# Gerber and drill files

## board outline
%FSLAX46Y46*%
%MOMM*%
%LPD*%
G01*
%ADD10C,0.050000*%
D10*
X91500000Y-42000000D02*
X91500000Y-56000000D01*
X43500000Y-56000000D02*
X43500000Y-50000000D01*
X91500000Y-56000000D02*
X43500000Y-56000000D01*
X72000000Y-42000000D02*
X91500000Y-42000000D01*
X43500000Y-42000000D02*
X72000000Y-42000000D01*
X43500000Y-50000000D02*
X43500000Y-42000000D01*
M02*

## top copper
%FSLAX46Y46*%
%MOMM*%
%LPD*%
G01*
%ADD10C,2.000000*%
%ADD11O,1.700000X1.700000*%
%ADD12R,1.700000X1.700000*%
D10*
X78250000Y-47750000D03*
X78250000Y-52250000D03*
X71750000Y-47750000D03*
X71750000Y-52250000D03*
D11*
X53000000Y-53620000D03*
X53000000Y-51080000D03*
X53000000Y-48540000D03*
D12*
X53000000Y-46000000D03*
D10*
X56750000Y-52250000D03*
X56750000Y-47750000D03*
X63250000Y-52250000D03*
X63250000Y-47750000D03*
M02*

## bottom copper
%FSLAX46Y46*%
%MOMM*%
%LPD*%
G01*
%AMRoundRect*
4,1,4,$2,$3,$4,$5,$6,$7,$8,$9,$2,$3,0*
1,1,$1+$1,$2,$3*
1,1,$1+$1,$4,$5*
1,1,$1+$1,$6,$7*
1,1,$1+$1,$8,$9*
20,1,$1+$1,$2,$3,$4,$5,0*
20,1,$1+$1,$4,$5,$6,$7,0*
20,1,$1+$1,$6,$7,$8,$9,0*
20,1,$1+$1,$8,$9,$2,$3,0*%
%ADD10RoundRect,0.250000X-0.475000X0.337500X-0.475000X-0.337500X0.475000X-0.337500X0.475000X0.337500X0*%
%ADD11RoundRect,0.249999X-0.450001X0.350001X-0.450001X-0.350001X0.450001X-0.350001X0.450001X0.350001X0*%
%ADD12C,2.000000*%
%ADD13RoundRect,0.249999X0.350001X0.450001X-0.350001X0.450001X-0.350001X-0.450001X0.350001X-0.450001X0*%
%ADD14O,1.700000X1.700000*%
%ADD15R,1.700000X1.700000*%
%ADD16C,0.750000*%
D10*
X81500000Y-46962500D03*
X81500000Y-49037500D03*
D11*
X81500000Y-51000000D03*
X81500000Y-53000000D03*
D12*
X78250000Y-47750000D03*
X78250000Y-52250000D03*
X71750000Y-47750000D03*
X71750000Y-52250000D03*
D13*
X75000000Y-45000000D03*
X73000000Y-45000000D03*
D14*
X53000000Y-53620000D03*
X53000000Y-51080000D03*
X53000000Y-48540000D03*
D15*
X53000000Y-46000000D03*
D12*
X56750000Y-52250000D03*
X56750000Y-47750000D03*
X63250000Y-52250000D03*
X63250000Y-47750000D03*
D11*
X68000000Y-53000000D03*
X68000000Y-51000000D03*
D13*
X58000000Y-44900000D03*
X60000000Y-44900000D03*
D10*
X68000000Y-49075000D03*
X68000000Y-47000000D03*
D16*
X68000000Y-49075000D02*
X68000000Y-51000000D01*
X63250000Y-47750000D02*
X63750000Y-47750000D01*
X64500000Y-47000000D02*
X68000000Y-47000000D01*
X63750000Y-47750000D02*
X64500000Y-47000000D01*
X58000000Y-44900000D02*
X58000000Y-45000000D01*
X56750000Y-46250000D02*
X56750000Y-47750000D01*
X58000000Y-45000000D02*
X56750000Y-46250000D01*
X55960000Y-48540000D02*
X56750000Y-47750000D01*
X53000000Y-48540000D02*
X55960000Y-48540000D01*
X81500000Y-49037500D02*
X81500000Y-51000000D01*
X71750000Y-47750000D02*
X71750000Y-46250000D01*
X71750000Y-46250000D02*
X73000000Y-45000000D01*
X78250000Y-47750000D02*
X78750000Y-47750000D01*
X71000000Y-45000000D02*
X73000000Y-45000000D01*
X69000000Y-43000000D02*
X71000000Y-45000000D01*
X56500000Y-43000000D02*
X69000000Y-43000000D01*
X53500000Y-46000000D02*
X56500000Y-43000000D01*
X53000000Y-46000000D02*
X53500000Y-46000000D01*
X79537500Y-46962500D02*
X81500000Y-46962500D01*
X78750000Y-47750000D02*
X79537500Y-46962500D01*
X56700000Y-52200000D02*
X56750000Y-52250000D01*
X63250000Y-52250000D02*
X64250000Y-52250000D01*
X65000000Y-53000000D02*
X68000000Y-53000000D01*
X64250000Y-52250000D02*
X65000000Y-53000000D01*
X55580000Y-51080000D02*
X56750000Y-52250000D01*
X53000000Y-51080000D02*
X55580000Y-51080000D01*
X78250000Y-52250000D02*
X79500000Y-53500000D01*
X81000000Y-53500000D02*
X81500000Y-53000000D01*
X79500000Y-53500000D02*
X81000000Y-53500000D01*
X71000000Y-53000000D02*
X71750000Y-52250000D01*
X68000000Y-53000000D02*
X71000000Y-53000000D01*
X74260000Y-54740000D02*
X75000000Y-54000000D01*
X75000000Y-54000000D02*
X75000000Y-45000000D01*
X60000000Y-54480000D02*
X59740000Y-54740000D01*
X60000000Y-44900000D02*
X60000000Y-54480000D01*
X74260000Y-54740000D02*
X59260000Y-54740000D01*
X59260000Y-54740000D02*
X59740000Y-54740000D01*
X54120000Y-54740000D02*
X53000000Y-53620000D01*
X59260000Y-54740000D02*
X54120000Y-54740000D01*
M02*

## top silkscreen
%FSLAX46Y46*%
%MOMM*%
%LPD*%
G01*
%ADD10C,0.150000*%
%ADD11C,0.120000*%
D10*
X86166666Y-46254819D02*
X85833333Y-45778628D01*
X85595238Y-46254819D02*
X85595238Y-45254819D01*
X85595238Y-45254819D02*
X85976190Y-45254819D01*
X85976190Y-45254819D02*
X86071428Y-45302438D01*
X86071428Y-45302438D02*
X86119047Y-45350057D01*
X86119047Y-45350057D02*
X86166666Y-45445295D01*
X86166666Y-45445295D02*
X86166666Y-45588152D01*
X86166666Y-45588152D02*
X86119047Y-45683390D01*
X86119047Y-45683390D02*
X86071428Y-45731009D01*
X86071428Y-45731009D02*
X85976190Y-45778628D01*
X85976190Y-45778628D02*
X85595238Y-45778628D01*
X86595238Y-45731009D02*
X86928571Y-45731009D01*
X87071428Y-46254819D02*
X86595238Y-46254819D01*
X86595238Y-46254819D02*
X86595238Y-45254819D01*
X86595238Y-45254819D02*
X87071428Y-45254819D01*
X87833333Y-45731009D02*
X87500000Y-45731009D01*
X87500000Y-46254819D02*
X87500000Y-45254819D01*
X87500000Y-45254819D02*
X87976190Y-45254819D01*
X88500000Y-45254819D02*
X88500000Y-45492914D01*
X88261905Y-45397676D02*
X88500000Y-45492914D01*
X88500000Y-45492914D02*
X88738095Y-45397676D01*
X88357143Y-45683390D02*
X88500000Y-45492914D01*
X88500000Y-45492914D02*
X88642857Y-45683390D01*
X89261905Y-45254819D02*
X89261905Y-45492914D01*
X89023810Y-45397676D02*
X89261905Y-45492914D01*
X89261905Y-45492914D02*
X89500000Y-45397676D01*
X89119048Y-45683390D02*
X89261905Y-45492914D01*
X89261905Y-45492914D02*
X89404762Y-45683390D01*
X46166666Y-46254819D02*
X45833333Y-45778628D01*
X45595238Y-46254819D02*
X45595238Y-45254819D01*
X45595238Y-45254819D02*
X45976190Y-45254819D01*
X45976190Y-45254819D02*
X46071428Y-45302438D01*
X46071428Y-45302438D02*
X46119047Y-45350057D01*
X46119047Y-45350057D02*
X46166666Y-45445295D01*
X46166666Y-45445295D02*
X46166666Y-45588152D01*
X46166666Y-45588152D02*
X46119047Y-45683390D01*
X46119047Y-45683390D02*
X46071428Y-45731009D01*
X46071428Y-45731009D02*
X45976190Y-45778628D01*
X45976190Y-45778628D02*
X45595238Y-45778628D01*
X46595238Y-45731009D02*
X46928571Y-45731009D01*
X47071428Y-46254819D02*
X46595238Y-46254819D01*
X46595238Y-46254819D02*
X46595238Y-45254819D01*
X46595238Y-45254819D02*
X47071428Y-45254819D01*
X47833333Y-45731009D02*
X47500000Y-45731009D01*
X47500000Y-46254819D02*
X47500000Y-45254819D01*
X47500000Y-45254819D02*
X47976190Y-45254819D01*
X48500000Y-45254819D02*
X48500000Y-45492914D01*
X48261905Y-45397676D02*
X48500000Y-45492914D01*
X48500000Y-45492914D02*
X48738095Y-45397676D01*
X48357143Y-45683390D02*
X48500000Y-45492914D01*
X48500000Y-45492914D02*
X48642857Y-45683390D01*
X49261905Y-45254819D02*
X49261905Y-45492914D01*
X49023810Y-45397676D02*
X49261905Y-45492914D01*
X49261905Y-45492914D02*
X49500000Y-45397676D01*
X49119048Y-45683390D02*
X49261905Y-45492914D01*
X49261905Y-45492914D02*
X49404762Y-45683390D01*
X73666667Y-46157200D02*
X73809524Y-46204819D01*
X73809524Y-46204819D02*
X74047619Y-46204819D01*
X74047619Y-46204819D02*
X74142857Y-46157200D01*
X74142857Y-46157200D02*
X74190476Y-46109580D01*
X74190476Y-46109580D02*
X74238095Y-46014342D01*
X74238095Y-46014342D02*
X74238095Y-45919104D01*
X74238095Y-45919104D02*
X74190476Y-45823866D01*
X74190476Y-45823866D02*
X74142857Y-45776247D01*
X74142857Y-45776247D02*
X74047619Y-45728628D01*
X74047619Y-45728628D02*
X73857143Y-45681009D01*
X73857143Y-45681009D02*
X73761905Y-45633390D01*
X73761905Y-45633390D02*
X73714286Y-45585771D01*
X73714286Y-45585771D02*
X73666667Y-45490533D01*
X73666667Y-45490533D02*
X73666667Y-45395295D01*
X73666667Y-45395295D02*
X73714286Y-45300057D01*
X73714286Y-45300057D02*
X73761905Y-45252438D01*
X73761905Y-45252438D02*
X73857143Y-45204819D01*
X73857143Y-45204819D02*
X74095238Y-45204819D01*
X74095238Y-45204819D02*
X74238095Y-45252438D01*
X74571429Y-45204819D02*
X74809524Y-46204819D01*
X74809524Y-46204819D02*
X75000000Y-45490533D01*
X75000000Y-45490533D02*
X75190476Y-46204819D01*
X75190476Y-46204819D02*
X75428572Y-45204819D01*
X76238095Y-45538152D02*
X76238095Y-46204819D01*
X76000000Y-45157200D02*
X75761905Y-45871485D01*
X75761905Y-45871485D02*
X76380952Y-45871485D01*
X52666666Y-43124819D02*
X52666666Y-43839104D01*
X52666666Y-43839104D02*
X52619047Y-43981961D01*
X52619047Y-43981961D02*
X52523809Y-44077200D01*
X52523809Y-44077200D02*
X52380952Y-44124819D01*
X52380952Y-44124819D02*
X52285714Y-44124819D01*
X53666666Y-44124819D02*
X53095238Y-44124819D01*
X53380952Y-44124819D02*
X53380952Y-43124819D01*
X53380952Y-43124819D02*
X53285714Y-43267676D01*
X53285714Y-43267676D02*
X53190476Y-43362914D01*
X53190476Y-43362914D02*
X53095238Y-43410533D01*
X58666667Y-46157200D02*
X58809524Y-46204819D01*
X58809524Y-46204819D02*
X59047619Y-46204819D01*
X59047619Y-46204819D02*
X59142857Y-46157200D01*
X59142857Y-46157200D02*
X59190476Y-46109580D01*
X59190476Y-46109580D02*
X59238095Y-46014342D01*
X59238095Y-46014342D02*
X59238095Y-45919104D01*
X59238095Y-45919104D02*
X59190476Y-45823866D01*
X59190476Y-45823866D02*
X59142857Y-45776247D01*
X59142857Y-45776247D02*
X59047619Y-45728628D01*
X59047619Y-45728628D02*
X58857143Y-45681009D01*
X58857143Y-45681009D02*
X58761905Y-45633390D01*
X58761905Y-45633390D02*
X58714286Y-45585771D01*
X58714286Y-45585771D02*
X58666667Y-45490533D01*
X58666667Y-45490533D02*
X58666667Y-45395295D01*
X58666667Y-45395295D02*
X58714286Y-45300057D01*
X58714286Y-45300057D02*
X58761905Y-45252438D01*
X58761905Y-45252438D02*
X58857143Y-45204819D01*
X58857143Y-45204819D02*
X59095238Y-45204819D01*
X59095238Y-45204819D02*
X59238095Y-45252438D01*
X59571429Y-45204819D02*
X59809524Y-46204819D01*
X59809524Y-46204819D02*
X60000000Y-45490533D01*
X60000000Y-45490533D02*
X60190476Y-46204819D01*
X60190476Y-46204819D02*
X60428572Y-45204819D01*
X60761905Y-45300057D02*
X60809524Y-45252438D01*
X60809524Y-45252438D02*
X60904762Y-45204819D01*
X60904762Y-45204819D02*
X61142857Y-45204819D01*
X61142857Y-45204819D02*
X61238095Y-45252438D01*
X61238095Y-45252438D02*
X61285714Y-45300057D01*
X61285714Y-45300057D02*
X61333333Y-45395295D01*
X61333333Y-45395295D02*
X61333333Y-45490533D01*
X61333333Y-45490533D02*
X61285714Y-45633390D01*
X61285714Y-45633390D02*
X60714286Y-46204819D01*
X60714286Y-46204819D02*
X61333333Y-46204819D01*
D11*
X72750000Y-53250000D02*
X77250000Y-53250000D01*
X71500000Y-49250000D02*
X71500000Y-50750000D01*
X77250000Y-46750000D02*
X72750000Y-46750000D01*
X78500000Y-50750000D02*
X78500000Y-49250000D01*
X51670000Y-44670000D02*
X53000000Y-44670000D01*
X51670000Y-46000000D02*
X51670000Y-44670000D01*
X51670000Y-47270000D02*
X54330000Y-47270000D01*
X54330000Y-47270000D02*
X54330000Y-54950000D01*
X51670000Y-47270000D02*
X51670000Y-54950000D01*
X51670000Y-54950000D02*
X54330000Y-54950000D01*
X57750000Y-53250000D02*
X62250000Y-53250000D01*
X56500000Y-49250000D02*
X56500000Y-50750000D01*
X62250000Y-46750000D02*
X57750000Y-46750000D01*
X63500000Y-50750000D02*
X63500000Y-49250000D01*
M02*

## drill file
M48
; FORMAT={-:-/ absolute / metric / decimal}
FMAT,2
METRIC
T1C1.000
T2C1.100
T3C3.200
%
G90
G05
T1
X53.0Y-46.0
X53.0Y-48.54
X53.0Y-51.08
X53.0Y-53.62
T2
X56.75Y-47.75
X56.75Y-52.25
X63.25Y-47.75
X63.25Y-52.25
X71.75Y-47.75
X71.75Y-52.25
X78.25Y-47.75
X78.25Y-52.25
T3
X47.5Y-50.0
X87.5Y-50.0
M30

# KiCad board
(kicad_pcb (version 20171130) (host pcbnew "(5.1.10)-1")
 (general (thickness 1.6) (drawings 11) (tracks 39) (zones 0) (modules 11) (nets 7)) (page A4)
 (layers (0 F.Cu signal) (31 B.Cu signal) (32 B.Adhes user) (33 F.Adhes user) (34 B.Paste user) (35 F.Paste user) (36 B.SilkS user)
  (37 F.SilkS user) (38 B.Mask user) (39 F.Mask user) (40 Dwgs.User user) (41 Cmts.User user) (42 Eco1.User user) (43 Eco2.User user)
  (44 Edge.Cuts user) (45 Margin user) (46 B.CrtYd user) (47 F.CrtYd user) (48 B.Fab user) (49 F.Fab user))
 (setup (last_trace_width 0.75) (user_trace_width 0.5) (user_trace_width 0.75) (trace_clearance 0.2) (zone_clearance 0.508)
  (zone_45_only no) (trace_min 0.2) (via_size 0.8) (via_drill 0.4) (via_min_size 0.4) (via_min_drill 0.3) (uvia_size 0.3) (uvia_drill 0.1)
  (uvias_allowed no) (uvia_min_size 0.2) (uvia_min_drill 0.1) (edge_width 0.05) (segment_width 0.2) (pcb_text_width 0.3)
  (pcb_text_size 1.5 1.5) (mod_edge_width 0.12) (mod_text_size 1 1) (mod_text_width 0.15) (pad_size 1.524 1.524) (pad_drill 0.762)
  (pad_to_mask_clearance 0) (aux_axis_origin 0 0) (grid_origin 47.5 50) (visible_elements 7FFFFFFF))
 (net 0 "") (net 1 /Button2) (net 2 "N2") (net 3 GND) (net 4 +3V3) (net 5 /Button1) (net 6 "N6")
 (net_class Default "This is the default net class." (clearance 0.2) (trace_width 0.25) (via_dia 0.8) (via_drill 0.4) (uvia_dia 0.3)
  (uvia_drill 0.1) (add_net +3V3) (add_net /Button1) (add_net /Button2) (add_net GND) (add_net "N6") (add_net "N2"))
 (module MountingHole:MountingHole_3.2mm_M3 (layer F.Cu) (at 87.5 50)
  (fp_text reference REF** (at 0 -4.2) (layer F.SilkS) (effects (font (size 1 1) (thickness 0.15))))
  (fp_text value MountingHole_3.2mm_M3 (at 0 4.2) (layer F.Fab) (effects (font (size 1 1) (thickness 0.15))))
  (pad 1 np_thru_hole circle (at 0 0) (size 3.2 3.2) (drill 3.2) (layers *.Cu *.Mask)))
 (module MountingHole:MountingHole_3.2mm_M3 (layer F.Cu) (at 47.5 50)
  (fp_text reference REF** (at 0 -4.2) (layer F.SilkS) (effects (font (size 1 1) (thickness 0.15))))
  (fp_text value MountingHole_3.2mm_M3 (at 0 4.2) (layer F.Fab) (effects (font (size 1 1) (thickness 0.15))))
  (pad 1 np_thru_hole circle (at 0 0) (size 3.2 3.2) (drill 3.2) (layers *.Cu *.Mask)))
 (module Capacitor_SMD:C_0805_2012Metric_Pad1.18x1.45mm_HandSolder (layer B.Cu) (at 81.5 48 270)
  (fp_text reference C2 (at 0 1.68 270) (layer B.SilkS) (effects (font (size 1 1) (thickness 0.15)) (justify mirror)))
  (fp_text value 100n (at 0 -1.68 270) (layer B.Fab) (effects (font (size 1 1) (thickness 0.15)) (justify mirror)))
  (pad 1 smd roundrect (at -1.0375 0 270) (size 1.175 1.45) (layers B.Cu B.Paste B.Mask) (roundrect_rratio 0.2127659574468085)
   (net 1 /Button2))
  (pad 2 smd roundrect (at 1.0375 0 270) (size 1.175 1.45) (layers B.Cu B.Paste B.Mask) (roundrect_rratio 0.2127659574468085) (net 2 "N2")))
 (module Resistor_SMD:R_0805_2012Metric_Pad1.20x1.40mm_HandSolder (layer B.Cu) (at 81.5 52 270)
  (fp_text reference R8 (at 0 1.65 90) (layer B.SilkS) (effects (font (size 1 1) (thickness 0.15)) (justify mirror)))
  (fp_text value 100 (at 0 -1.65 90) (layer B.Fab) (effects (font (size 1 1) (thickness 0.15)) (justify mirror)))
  (pad 1 smd roundrect (at -1 0 270) (size 1.2 1.4) (layers B.Cu B.Paste B.Mask) (roundrect_rratio 0.2083325) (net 2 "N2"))
  (pad 2 smd roundrect (at 1 0 270) (size 1.2 1.4) (layers B.Cu B.Paste B.Mask) (roundrect_rratio 0.2083325) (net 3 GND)))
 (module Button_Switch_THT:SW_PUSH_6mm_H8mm (layer F.Cu) (at 71.75 47.75)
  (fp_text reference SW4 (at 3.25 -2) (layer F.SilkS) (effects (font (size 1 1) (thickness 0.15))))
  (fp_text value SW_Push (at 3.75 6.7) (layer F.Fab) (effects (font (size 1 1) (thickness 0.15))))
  (fp_line (start 1 5.5) (end 5.5 5.5) (layer F.SilkS) (width 0.12))
  (fp_line (start -0.25 1.5) (end -0.25 3) (layer F.SilkS) (width 0.12))
  (fp_line (start 5.5 -1) (end 1 -1) (layer F.SilkS) (width 0.12))
  (fp_line (start 6.75 3) (end 6.75 1.5) (layer F.SilkS) (width 0.12))
  (pad 1 thru_hole circle (at 6.5 0 90) (size 2 2) (drill 1.1) (layers *.Cu *.Mask) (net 1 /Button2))
  (pad 2 thru_hole circle (at 6.5 4.5 90) (size 2 2) (drill 1.1) (layers *.Cu *.Mask) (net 3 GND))
  (pad 1 thru_hole circle (at 0 0 90) (size 2 2) (drill 1.1) (layers *.Cu *.Mask) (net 1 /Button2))
  (pad 2 thru_hole circle (at 0 4.5 90) (size 2 2) (drill 1.1) (layers *.Cu *.Mask) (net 3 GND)))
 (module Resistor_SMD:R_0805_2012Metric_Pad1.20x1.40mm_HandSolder (layer B.Cu) (at 74 45 180)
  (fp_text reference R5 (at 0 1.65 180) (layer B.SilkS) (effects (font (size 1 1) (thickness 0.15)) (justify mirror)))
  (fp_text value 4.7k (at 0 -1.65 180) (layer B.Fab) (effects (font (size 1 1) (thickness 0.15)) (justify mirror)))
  (pad 1 smd roundrect (at -1 0 180) (size 1.2 1.4) (layers B.Cu B.Paste B.Mask) (roundrect_rratio 0.2083325) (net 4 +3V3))
  (pad 2 smd roundrect (at 1 0 180) (size 1.2 1.4) (layers B.Cu B.Paste B.Mask) (roundrect_rratio 0.2083325) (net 1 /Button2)))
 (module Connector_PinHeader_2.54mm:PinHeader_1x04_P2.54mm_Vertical (layer F.Cu) (at 53 46)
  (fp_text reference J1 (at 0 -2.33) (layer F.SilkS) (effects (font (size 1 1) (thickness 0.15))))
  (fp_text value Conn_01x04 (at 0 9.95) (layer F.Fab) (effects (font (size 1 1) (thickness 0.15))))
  (fp_line (start -1.33 -1.33) (end 0 -1.33) (layer F.SilkS) (width 0.12))
  (fp_line (start -1.33 0) (end -1.33 -1.33) (layer F.SilkS) (width 0.12))
  (fp_line (start -1.33 1.27) (end 1.33 1.27) (layer F.SilkS) (width 0.12))
  (fp_line (start 1.33 1.27) (end 1.33 8.95) (layer F.SilkS) (width 0.12))
  (fp_line (start -1.33 1.27) (end -1.33 8.95) (layer F.SilkS) (width 0.12))
  (fp_line (start -1.33 8.95) (end 1.33 8.95) (layer F.SilkS) (width 0.12))
  (pad 4 thru_hole oval (at 0 7.62) (size 1.7 1.7) (drill 1) (layers *.Cu *.Mask) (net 4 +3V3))
  (pad 3 thru_hole oval (at 0 5.08) (size 1.7 1.7) (drill 1) (layers *.Cu *.Mask) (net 3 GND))
  (pad 2 thru_hole oval (at 0 2.54) (size 1.7 1.7) (drill 1) (layers *.Cu *.Mask) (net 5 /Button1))
  (pad 1 thru_hole rect (at 0 0) (size 1.7 1.7) (drill 1) (layers *.Cu *.Mask) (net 1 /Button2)))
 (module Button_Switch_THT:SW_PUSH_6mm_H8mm (layer F.Cu) (at 56.75 47.75)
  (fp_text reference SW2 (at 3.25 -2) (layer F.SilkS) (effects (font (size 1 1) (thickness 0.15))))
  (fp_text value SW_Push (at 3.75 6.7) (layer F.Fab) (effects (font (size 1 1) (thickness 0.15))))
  (fp_line (start 1 5.5) (end 5.5 5.5) (layer F.SilkS) (width 0.12))
  (fp_line (start -0.25 1.5) (end -0.25 3) (layer F.SilkS) (width 0.12))
  (fp_line (start 5.5 -1) (end 1 -1) (layer F.SilkS) (width 0.12))
  (fp_line (start 6.75 3) (end 6.75 1.5) (layer F.SilkS) (width 0.12))
  (pad 2 thru_hole circle (at 0 4.5 90) (size 2 2) (drill 1.1) (layers *.Cu *.Mask) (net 3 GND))
  (pad 1 thru_hole circle (at 0 0 90) (size 2 2) (drill 1.1) (layers *.Cu *.Mask) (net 5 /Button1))
  (pad 2 thru_hole circle (at 6.5 4.5 90) (size 2 2) (drill 1.1) (layers *.Cu *.Mask) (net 3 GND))
  (pad 1 thru_hole circle (at 6.5 0 90) (size 2 2) (drill 1.1) (layers *.Cu *.Mask) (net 5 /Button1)))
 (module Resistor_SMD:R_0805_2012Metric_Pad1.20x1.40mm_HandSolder (layer B.Cu) (at 68 52 270)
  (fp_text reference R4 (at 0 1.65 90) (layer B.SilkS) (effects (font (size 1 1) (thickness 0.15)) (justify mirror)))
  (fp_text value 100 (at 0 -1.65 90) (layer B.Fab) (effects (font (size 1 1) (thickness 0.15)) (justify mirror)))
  (pad 2 smd roundrect (at 1 0 270) (size 1.2 1.4) (layers B.Cu B.Paste B.Mask) (roundrect_rratio 0.2083325) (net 3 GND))
  (pad 1 smd roundrect (at -1 0 270) (size 1.2 1.4) (layers B.Cu B.Paste B.Mask) (roundrect_rratio 0.2083325) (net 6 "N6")))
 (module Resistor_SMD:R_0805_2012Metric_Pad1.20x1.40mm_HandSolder (layer B.Cu) (at 59 44.9 180)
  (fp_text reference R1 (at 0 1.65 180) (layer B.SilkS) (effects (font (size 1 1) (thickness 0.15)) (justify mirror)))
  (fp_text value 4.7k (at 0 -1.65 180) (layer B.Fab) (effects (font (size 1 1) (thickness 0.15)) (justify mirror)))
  (pad 2 smd roundrect (at 1 0 180) (size 1.2 1.4) (layers B.Cu B.Paste B.Mask) (roundrect_rratio 0.2083325) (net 5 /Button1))
  (pad 1 smd roundrect (at -1 0 180) (size 1.2 1.4) (layers B.Cu B.Paste B.Mask) (roundrect_rratio 0.2083325) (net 4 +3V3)))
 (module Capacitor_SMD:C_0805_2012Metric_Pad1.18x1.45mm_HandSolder (layer B.Cu) (at 68 48.0375 270)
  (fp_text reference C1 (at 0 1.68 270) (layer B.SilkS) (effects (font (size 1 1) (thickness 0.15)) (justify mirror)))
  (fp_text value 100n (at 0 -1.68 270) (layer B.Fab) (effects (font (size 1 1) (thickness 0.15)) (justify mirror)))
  (pad 2 smd roundrect (at 1.0375 0 270) (size 1.175 1.45) (layers B.Cu B.Paste B.Mask) (roundrect_rratio 0.2127659574468085) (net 6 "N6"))
  (pad 1 smd roundrect (at -1.0375 0 270) (size 1.175 1.45) (layers B.Cu B.Paste B.Mask) (roundrect_rratio 0.2127659574468085)
   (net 5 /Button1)))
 (gr_line (start 91.5 42) (end 91.5 56) (layer Edge.Cuts) (width 0.05))
 (gr_line (start 43.5 56) (end 43.5 50) (layer Edge.Cuts) (width 0.05))
 (gr_line (start 91.5 56) (end 43.5 56) (layer Edge.Cuts) (width 0.05))
 (gr_line (start 72 42) (end 91.5 42) (layer Edge.Cuts) (width 0.05))
 (gr_line (start 43.5 42) (end 72 42) (layer Edge.Cuts) (width 0.05))
 (gr_line (start 43.5 50) (end 43.5 42) (layer Edge.Cuts) (width 0.05))
 (segment (start 68 49.075) (end 68 51) (width 0.75) (layer B.Cu) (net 6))
 (segment (start 63.25 47.75) (end 63.75 47.75) (width 0.75) (layer B.Cu) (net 5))
 (segment (start 64.5 47) (end 68 47) (width 0.75) (layer B.Cu) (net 5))
 (segment (start 63.75 47.75) (end 64.5 47) (width 0.75) (layer B.Cu) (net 5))
 (segment (start 58 44.9) (end 58 45) (width 0.75) (layer B.Cu) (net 5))
 (segment (start 56.75 46.25) (end 56.75 47.75) (width 0.75) (layer B.Cu) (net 5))
 (segment (start 58 45) (end 56.75 46.25) (width 0.75) (layer B.Cu) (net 5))
 (segment (start 55.96 48.54) (end 56.75 47.75) (width 0.75) (layer B.Cu) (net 5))
 (segment (start 53 48.54) (end 55.96 48.54) (width 0.75) (layer B.Cu) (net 5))
 (segment (start 81.5 49.0375) (end 81.5 51) (width 0.75) (layer B.Cu) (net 2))
 (segment (start 71.75 47.75) (end 71.75 46.25) (width 0.75) (layer B.Cu) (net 1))
 (segment (start 71.75 46.25) (end 73 45) (width 0.75) (layer B.Cu) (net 1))
 (segment (start 78.25 47.75) (end 78.75 47.75) (width 0.75) (layer B.Cu) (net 1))
 (segment (start 71 45) (end 73 45) (width 0.75) (layer B.Cu) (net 1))
 (segment (start 69 43) (end 71 45) (width 0.75) (layer B.Cu) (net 1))
 (segment (start 56.5 43) (end 69 43) (width 0.75) (layer B.Cu) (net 1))
 (segment (start 53.5 46) (end 56.5 43) (width 0.75) (layer B.Cu) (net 1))
 (segment (start 53 46) (end 53.5 46) (width 0.75) (layer B.Cu) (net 1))
 (segment (start 79.5375 46.9625) (end 81.5 46.9625) (width 0.75) (layer B.Cu) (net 1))
 (segment (start 78.75 47.75) (end 79.5375 46.9625) (width 0.75) (layer B.Cu) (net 1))
 (segment (start 56.7 52.2) (end 56.75 52.25) (width 0.75) (layer B.Cu) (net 3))
 (segment (start 63.25 52.25) (end 64.25 52.25) (width 0.75) (layer B.Cu) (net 3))
 (segment (start 65 53) (end 68 53) (width 0.75) (layer B.Cu) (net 3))
 (segment (start 64.25 52.25) (end 65 53) (width 0.75) (layer B.Cu) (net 3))
 (segment (start 55.58 51.08) (end 56.75 52.25) (width 0.75) (layer B.Cu) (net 3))
 (segment (start 53 51.08) (end 55.58 51.08) (width 0.75) (layer B.Cu) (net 3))
 (segment (start 78.25 52.25) (end 79.5 53.5) (width 0.75) (layer B.Cu) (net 3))
 (segment (start 81 53.5) (end 81.5 53) (width 0.75) (layer B.Cu) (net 3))
 (segment (start 79.5 53.5) (end 81 53.5) (width 0.75) (layer B.Cu) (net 3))
 (segment (start 71 53) (end 71.75 52.25) (width 0.75) (layer B.Cu) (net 3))
 (segment (start 68 53) (end 71 53) (width 0.75) (layer B.Cu) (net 3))
 (segment (start 74.26 54.74) (end 75 54) (width 0.75) (layer B.Cu) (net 4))
 (segment (start 75 54) (end 75 45) (width 0.75) (layer B.Cu) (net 4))
 (segment (start 60 54.48) (end 59.74 54.74) (width 0.75) (layer B.Cu) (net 4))
 (segment (start 60 44.9) (end 60 54.48) (width 0.75) (layer B.Cu) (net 4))
 (segment (start 74.26 54.74) (end 59.26 54.74) (width 0.75) (layer B.Cu) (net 4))
 (segment (start 59.26 54.74) (end 59.74 54.74) (width 0.75) (layer B.Cu) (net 4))
 (segment (start 54.12 54.74) (end 53 53.62) (width 0.75) (layer B.Cu) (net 4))
 (segment (start 59.26 54.74) (end 54.12 54.74) (width 0.75) (layer B.Cu) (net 4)))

